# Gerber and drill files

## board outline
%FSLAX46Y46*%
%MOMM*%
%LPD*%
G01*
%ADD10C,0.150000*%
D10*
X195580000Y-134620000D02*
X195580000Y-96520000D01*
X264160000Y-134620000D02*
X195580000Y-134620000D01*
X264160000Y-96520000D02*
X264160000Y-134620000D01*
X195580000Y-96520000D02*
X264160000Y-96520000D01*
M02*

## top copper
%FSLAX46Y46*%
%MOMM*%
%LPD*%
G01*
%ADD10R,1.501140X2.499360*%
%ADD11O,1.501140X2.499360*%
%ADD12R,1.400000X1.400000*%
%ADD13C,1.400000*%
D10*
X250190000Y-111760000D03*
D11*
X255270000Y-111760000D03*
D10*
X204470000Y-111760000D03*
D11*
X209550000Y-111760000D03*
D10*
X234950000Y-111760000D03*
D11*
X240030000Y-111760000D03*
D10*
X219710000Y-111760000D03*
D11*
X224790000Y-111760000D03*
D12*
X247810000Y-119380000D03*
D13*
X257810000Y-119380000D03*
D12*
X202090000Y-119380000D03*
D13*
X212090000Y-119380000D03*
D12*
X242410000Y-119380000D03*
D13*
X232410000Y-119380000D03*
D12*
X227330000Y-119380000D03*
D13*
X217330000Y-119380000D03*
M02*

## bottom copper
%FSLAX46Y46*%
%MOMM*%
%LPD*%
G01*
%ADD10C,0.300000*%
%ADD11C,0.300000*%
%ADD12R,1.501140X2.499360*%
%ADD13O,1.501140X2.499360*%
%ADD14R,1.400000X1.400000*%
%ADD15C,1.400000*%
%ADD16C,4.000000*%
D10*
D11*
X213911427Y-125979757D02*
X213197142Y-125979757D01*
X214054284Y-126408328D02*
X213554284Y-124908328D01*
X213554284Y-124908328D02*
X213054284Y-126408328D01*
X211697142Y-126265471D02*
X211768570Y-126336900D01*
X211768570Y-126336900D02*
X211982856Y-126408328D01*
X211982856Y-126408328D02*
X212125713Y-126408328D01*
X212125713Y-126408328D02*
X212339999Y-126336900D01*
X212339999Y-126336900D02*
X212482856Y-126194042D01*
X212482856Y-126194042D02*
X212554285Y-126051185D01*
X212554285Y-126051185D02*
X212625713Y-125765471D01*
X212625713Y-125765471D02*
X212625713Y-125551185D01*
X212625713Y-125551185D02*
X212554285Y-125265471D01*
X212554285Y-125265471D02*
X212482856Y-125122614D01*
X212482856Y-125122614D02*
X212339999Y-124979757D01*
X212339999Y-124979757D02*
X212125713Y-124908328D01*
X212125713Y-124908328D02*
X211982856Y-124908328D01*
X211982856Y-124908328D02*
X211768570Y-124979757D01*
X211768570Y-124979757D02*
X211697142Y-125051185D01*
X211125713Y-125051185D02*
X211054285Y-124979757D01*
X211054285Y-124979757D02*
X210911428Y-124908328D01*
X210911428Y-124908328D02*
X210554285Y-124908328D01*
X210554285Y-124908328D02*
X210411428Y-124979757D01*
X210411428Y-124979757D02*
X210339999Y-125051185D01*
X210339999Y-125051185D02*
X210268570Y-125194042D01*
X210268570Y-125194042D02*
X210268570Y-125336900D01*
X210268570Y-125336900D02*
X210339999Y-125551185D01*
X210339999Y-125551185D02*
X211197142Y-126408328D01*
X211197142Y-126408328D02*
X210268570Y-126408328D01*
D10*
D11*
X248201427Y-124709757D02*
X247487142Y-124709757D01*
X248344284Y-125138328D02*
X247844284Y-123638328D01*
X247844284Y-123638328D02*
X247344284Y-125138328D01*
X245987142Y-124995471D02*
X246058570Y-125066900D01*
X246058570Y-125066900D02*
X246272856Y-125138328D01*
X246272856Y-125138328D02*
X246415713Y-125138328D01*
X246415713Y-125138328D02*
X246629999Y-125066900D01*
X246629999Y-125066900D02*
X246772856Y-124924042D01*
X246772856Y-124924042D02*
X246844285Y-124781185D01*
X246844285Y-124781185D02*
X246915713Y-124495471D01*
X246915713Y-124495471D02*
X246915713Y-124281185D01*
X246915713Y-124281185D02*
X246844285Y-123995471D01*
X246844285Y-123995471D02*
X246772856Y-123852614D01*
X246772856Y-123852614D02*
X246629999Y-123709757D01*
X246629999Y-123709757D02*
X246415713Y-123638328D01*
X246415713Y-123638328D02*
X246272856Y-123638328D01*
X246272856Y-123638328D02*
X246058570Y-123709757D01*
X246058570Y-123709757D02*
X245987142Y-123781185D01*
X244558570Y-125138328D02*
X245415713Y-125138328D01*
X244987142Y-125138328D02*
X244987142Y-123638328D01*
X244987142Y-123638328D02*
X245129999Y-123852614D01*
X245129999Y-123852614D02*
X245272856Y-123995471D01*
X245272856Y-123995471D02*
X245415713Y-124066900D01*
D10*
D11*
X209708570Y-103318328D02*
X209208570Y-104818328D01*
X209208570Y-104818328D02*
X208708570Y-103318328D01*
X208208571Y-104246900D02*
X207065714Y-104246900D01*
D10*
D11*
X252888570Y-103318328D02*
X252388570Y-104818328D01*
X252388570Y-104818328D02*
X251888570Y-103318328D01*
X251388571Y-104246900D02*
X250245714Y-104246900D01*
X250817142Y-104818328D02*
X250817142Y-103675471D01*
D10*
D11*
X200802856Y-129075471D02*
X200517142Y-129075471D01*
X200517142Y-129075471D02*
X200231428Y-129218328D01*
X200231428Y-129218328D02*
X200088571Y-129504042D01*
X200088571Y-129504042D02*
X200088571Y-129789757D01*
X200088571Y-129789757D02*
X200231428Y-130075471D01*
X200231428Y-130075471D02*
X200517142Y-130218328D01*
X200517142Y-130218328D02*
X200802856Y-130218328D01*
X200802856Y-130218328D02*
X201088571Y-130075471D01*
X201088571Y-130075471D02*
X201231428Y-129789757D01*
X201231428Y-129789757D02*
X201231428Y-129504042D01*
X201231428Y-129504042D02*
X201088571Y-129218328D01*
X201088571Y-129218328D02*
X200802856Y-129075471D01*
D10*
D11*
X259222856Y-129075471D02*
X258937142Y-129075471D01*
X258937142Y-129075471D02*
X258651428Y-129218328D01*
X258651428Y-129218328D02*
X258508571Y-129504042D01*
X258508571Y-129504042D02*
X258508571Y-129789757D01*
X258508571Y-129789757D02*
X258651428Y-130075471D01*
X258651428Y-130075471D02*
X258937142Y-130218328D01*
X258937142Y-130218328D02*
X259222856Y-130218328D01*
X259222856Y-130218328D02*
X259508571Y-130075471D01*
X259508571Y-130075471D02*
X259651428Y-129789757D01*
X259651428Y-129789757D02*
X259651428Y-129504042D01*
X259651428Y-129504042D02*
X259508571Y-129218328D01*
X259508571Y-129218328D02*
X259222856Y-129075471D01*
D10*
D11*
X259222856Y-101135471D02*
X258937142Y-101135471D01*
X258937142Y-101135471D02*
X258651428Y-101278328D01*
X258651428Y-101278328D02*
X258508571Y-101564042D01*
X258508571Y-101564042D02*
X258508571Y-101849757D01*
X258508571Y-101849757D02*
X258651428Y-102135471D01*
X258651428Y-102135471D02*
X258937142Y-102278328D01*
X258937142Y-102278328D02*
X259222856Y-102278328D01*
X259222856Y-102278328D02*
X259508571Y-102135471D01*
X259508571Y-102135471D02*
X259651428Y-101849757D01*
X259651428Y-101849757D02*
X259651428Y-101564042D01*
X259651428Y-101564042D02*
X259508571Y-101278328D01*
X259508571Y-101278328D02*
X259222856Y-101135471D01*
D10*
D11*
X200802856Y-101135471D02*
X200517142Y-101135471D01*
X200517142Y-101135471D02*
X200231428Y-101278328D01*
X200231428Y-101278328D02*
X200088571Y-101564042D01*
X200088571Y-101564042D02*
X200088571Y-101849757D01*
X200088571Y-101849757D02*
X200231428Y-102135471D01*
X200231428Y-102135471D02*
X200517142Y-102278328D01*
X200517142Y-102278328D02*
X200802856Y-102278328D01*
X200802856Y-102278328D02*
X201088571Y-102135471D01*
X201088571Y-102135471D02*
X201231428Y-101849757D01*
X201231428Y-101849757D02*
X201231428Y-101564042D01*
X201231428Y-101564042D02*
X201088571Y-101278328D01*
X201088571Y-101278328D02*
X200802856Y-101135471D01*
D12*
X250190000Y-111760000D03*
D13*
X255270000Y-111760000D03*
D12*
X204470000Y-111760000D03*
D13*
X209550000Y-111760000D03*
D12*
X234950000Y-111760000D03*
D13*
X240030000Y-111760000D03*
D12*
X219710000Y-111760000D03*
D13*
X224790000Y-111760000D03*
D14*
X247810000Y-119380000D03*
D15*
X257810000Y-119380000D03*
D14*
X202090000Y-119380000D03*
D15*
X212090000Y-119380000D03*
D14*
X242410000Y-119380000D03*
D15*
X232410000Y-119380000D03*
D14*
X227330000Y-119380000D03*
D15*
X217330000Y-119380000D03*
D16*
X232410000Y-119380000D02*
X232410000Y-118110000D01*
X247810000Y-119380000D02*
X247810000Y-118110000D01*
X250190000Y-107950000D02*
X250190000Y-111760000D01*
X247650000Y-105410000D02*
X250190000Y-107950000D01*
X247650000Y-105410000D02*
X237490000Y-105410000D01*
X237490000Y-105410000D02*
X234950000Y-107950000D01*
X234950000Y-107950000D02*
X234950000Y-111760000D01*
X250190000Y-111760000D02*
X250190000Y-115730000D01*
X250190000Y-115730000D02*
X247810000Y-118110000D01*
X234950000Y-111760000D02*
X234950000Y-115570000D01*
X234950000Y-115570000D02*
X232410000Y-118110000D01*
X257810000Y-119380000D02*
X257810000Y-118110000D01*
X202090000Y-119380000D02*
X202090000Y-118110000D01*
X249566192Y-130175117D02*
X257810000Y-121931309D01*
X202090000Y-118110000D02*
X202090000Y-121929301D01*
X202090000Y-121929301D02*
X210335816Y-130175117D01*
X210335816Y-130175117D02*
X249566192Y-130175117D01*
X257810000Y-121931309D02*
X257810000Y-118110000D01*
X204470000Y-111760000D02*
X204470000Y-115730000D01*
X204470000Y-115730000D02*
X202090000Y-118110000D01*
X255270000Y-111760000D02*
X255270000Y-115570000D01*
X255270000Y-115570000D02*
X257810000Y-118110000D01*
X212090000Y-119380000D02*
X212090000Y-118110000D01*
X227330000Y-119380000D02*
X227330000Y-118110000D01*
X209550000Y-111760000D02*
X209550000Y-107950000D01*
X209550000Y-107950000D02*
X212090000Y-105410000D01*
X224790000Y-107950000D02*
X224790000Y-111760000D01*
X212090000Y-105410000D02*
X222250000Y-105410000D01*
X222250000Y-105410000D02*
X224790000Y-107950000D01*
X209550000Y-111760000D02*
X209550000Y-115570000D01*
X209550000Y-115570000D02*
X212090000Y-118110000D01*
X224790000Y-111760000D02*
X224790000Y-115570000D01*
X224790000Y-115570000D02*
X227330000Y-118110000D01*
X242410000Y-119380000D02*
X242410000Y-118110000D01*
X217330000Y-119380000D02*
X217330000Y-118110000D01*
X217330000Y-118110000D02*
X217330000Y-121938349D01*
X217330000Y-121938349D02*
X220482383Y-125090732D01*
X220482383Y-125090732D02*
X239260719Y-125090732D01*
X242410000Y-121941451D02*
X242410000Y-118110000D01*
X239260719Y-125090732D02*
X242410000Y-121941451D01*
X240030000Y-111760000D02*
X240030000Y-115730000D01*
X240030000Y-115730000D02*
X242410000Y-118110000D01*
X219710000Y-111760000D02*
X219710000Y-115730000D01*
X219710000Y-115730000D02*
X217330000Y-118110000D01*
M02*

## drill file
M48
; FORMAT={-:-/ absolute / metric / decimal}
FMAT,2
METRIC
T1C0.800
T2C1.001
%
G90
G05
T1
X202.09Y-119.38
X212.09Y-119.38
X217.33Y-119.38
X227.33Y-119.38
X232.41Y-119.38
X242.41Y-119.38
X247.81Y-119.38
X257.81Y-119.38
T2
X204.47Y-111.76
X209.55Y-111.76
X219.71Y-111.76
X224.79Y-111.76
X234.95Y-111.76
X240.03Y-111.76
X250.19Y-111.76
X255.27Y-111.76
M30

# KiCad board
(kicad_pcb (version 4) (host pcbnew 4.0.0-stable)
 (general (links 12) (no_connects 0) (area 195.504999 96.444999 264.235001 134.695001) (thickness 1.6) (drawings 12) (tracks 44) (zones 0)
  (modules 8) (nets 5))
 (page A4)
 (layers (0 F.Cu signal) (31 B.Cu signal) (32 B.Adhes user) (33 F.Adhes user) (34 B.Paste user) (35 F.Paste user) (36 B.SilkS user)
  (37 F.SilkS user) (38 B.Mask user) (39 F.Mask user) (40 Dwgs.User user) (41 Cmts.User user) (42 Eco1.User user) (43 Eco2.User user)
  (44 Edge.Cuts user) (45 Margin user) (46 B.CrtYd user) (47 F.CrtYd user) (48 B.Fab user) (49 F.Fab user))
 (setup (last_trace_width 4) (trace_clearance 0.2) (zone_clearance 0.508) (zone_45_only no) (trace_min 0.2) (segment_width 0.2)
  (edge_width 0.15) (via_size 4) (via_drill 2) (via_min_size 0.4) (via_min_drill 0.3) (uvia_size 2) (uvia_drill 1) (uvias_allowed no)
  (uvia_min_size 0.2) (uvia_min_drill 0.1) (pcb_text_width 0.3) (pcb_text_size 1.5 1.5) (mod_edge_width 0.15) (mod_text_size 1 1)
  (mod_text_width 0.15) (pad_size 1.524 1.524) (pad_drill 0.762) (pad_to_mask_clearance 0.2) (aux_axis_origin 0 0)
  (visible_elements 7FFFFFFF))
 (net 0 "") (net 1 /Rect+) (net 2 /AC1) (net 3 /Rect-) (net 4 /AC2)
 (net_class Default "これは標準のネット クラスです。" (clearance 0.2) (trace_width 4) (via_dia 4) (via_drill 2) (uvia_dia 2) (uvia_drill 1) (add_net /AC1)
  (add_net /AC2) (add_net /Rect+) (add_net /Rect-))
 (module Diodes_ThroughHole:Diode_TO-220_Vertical (layer F.Cu) (at 250.19 111.76)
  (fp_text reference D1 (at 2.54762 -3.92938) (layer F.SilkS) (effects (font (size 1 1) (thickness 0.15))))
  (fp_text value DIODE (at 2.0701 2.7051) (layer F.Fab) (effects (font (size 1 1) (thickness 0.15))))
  (pad 1 thru_hole rect (at 0 0 90) (size 2.49936 1.50114) (drill 1.00076) (layers *.Cu *.Mask F.SilkS) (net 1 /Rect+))
  (pad 2 thru_hole oval (at 5.08 0 90) (size 2.49936 1.50114) (drill 1.00076) (layers *.Cu *.Mask F.SilkS) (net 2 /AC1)))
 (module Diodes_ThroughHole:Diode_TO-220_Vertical (layer F.Cu) (at 204.47 111.76)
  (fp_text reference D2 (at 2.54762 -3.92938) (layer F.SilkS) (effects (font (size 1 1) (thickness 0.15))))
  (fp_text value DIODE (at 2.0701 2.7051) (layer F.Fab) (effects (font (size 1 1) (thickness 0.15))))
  (pad 1 thru_hole rect (at 0 0 90) (size 2.49936 1.50114) (drill 1.00076) (layers *.Cu *.Mask F.SilkS) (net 2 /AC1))
  (pad 2 thru_hole oval (at 5.08 0 90) (size 2.49936 1.50114) (drill 1.00076) (layers *.Cu *.Mask F.SilkS) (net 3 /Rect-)))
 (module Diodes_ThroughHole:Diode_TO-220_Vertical (layer F.Cu) (at 234.95 111.76)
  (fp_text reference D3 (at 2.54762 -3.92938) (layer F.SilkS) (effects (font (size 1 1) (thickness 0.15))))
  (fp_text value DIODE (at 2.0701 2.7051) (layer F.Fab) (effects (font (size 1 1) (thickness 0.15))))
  (pad 1 thru_hole rect (at 0 0 90) (size 2.49936 1.50114) (drill 1.00076) (layers *.Cu *.Mask F.SilkS) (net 1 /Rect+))
  (pad 2 thru_hole oval (at 5.08 0 90) (size 2.49936 1.50114) (drill 1.00076) (layers *.Cu *.Mask F.SilkS) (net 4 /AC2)))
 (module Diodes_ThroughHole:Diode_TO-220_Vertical (layer F.Cu) (at 219.71 111.76)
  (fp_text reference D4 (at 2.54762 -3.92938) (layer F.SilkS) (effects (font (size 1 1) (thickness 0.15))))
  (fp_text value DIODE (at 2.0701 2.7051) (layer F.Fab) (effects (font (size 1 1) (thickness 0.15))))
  (pad 1 thru_hole rect (at 0 0 90) (size 2.49936 1.50114) (drill 1.00076) (layers *.Cu *.Mask F.SilkS) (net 4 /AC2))
  (pad 2 thru_hole oval (at 5.08 0 90) (size 2.49936 1.50114) (drill 1.00076) (layers *.Cu *.Mask F.SilkS) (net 3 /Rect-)))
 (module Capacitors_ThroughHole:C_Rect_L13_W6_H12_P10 (layer F.Cu) (at 247.81 119.38)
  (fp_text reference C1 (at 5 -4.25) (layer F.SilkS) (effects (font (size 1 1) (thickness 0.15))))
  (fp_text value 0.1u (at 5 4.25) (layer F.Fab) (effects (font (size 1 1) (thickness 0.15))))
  (pad 1 thru_hole rect (at 0 0) (size 1.4 1.4) (drill 0.8) (layers *.Cu *.Mask F.SilkS) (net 1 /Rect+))
  (pad 2 thru_hole circle (at 10 0) (size 1.4 1.4) (drill 0.8) (layers *.Cu *.Mask F.SilkS) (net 2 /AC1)))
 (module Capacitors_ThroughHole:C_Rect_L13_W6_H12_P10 (layer F.Cu) (at 202.09 119.38)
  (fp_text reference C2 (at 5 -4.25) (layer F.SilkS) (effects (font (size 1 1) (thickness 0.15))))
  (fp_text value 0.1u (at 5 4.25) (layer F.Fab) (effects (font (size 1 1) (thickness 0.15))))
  (pad 1 thru_hole rect (at 0 0) (size 1.4 1.4) (drill 0.8) (layers *.Cu *.Mask F.SilkS) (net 2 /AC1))
  (pad 2 thru_hole circle (at 10 0) (size 1.4 1.4) (drill 0.8) (layers *.Cu *.Mask F.SilkS) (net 3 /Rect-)))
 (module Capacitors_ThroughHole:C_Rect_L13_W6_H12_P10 (layer F.Cu) (at 242.41 119.38 180)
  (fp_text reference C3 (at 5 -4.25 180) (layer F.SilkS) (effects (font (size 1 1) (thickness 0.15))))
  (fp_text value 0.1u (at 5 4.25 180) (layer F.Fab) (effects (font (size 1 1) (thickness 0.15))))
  (pad 1 thru_hole rect (at 0 0 180) (size 1.4 1.4) (drill 0.8) (layers *.Cu *.Mask F.SilkS) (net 4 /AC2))
  (pad 2 thru_hole circle (at 10 0 180) (size 1.4 1.4) (drill 0.8) (layers *.Cu *.Mask F.SilkS) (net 1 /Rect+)))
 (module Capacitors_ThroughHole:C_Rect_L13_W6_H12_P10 (layer F.Cu) (at 227.33 119.38 180)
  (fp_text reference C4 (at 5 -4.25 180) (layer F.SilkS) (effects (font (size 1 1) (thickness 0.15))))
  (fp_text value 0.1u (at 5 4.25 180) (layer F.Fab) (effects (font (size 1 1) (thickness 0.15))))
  (pad 1 thru_hole rect (at 0 0 180) (size 1.4 1.4) (drill 0.8) (layers *.Cu *.Mask F.SilkS) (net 3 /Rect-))
  (pad 2 thru_hole circle (at 10 0 180) (size 1.4 1.4) (drill 0.8) (layers *.Cu *.Mask F.SilkS) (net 4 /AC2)))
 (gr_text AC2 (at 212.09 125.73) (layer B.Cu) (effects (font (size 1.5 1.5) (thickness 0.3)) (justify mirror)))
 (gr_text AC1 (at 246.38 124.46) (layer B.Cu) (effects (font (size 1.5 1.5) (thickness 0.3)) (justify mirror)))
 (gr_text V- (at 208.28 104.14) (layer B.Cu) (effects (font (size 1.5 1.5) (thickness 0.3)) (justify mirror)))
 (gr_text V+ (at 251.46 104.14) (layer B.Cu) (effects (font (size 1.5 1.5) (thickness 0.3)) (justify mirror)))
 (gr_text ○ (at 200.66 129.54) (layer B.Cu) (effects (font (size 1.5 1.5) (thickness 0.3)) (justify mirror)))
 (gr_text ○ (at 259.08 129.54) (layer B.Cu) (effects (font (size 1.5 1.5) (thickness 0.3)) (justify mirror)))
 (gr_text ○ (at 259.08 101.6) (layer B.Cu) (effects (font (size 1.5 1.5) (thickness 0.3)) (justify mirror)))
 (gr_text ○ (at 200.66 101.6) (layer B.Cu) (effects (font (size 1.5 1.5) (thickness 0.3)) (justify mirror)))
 (gr_line (start 195.58 134.62) (end 195.58 96.52) (layer Edge.Cuts) (width 0.15))
 (gr_line (start 264.16 134.62) (end 195.58 134.62) (layer Edge.Cuts) (width 0.15))
 (gr_line (start 264.16 96.52) (end 264.16 134.62) (layer Edge.Cuts) (width 0.15))
 (gr_line (start 195.58 96.52) (end 264.16 96.52) (layer Edge.Cuts) (width 0.15))
 (segment (start 232.41 119.38) (end 232.41 118.11) (width 4) (layer B.Cu) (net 1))
 (segment (start 247.81 119.38) (end 247.81 118.11) (width 4) (layer B.Cu) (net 1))
 (segment (start 250.19 107.95) (end 250.19 111.76) (width 4) (layer B.Cu) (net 1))
 (segment (start 247.65 105.41) (end 250.19 107.95) (width 4) (layer B.Cu) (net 1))
 (segment (start 247.65 105.41) (end 237.49 105.41) (width 4) (layer B.Cu) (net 1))
 (segment (start 237.49 105.41) (end 234.95 107.95) (width 4) (layer B.Cu) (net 1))
 (segment (start 234.95 107.95) (end 234.95 111.76) (width 4) (layer B.Cu) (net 1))
 (segment (start 250.19 111.76) (end 250.19 115.73) (width 4) (layer B.Cu) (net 1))
 (segment (start 250.19 115.73) (end 247.81 118.11) (width 4) (layer B.Cu) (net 1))
 (segment (start 234.95 111.76) (end 234.95 115.57) (width 4) (layer B.Cu) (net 1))
 (segment (start 234.95 115.57) (end 232.41 118.11) (width 4) (layer B.Cu) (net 1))
 (segment (start 257.81 119.38) (end 257.81 118.11) (width 4) (layer B.Cu) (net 2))
 (segment (start 202.09 119.38) (end 202.09 118.11) (width 4) (layer B.Cu) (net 2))
 (segment (start 249.566192 130.175117) (end 257.81 121.931309) (width 4) (layer B.Cu) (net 2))
 (segment (start 202.09 118.11) (end 202.09 121.929301) (width 4) (layer B.Cu) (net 2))
 (segment (start 202.09 121.929301) (end 210.335816 130.175117) (width 4) (layer B.Cu) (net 2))
 (segment (start 210.335816 130.175117) (end 249.566192 130.175117) (width 4) (layer B.Cu) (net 2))
 (segment (start 257.81 121.931309) (end 257.81 118.11) (width 4) (layer B.Cu) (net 2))
 (segment (start 204.47 111.76) (end 204.47 115.73) (width 4) (layer B.Cu) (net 2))
 (segment (start 204.47 115.73) (end 202.09 118.11) (width 4) (layer B.Cu) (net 2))
 (segment (start 255.27 111.76) (end 255.27 115.57) (width 4) (layer B.Cu) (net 2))
 (segment (start 255.27 115.57) (end 257.81 118.11) (width 4) (layer B.Cu) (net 2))
 (segment (start 212.09 119.38) (end 212.09 118.11) (width 4) (layer B.Cu) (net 3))
 (segment (start 227.33 119.38) (end 227.33 118.11) (width 4) (layer B.Cu) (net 3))
 (segment (start 209.55 111.76) (end 209.55 107.95) (width 4) (layer B.Cu) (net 3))
 (segment (start 209.55 107.95) (end 212.09 105.41) (width 4) (layer B.Cu) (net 3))
 (segment (start 224.79 107.95) (end 224.79 111.76) (width 4) (layer B.Cu) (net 3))
 (segment (start 212.09 105.41) (end 222.25 105.41) (width 4) (layer B.Cu) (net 3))
 (segment (start 222.25 105.41) (end 224.79 107.95) (width 4) (layer B.Cu) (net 3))
 (segment (start 209.55 111.76) (end 209.55 115.57) (width 4) (layer B.Cu) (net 3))
 (segment (start 209.55 115.57) (end 212.09 118.11) (width 4) (layer B.Cu) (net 3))
 (segment (start 224.79 111.76) (end 224.79 115.57) (width 4) (layer B.Cu) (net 3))
 (segment (start 224.79 115.57) (end 227.33 118.11) (width 4) (layer B.Cu) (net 3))
 (segment (start 242.41 119.38) (end 242.41 118.11) (width 4) (layer B.Cu) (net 4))
 (segment (start 217.33 119.38) (end 217.33 118.11) (width 4) (layer B.Cu) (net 4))
 (segment (start 217.33 118.11) (end 217.33 121.938349) (width 4) (layer B.Cu) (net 4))
 (segment (start 217.33 121.938349) (end 220.482383 125.090732) (width 4) (layer B.Cu) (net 4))
 (segment (start 220.482383 125.090732) (end 239.260719 125.090732) (width 4) (layer B.Cu) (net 4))
 (segment (start 242.41 121.941451) (end 242.41 118.11) (width 4) (layer B.Cu) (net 4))
 (segment (start 239.260719 125.090732) (end 242.41 121.941451) (width 4) (layer B.Cu) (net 4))
 (segment (start 240.03 111.76) (end 240.03 115.73) (width 4) (layer B.Cu) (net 4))
 (segment (start 240.03 115.73) (end 242.41 118.11) (width 4) (layer B.Cu) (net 4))
 (segment (start 219.71 111.76) (end 219.71 115.73) (width 4) (layer B.Cu) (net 4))
 (segment (start 219.71 115.73) (end 217.33 118.11) (width 4) (layer B.Cu) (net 4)))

